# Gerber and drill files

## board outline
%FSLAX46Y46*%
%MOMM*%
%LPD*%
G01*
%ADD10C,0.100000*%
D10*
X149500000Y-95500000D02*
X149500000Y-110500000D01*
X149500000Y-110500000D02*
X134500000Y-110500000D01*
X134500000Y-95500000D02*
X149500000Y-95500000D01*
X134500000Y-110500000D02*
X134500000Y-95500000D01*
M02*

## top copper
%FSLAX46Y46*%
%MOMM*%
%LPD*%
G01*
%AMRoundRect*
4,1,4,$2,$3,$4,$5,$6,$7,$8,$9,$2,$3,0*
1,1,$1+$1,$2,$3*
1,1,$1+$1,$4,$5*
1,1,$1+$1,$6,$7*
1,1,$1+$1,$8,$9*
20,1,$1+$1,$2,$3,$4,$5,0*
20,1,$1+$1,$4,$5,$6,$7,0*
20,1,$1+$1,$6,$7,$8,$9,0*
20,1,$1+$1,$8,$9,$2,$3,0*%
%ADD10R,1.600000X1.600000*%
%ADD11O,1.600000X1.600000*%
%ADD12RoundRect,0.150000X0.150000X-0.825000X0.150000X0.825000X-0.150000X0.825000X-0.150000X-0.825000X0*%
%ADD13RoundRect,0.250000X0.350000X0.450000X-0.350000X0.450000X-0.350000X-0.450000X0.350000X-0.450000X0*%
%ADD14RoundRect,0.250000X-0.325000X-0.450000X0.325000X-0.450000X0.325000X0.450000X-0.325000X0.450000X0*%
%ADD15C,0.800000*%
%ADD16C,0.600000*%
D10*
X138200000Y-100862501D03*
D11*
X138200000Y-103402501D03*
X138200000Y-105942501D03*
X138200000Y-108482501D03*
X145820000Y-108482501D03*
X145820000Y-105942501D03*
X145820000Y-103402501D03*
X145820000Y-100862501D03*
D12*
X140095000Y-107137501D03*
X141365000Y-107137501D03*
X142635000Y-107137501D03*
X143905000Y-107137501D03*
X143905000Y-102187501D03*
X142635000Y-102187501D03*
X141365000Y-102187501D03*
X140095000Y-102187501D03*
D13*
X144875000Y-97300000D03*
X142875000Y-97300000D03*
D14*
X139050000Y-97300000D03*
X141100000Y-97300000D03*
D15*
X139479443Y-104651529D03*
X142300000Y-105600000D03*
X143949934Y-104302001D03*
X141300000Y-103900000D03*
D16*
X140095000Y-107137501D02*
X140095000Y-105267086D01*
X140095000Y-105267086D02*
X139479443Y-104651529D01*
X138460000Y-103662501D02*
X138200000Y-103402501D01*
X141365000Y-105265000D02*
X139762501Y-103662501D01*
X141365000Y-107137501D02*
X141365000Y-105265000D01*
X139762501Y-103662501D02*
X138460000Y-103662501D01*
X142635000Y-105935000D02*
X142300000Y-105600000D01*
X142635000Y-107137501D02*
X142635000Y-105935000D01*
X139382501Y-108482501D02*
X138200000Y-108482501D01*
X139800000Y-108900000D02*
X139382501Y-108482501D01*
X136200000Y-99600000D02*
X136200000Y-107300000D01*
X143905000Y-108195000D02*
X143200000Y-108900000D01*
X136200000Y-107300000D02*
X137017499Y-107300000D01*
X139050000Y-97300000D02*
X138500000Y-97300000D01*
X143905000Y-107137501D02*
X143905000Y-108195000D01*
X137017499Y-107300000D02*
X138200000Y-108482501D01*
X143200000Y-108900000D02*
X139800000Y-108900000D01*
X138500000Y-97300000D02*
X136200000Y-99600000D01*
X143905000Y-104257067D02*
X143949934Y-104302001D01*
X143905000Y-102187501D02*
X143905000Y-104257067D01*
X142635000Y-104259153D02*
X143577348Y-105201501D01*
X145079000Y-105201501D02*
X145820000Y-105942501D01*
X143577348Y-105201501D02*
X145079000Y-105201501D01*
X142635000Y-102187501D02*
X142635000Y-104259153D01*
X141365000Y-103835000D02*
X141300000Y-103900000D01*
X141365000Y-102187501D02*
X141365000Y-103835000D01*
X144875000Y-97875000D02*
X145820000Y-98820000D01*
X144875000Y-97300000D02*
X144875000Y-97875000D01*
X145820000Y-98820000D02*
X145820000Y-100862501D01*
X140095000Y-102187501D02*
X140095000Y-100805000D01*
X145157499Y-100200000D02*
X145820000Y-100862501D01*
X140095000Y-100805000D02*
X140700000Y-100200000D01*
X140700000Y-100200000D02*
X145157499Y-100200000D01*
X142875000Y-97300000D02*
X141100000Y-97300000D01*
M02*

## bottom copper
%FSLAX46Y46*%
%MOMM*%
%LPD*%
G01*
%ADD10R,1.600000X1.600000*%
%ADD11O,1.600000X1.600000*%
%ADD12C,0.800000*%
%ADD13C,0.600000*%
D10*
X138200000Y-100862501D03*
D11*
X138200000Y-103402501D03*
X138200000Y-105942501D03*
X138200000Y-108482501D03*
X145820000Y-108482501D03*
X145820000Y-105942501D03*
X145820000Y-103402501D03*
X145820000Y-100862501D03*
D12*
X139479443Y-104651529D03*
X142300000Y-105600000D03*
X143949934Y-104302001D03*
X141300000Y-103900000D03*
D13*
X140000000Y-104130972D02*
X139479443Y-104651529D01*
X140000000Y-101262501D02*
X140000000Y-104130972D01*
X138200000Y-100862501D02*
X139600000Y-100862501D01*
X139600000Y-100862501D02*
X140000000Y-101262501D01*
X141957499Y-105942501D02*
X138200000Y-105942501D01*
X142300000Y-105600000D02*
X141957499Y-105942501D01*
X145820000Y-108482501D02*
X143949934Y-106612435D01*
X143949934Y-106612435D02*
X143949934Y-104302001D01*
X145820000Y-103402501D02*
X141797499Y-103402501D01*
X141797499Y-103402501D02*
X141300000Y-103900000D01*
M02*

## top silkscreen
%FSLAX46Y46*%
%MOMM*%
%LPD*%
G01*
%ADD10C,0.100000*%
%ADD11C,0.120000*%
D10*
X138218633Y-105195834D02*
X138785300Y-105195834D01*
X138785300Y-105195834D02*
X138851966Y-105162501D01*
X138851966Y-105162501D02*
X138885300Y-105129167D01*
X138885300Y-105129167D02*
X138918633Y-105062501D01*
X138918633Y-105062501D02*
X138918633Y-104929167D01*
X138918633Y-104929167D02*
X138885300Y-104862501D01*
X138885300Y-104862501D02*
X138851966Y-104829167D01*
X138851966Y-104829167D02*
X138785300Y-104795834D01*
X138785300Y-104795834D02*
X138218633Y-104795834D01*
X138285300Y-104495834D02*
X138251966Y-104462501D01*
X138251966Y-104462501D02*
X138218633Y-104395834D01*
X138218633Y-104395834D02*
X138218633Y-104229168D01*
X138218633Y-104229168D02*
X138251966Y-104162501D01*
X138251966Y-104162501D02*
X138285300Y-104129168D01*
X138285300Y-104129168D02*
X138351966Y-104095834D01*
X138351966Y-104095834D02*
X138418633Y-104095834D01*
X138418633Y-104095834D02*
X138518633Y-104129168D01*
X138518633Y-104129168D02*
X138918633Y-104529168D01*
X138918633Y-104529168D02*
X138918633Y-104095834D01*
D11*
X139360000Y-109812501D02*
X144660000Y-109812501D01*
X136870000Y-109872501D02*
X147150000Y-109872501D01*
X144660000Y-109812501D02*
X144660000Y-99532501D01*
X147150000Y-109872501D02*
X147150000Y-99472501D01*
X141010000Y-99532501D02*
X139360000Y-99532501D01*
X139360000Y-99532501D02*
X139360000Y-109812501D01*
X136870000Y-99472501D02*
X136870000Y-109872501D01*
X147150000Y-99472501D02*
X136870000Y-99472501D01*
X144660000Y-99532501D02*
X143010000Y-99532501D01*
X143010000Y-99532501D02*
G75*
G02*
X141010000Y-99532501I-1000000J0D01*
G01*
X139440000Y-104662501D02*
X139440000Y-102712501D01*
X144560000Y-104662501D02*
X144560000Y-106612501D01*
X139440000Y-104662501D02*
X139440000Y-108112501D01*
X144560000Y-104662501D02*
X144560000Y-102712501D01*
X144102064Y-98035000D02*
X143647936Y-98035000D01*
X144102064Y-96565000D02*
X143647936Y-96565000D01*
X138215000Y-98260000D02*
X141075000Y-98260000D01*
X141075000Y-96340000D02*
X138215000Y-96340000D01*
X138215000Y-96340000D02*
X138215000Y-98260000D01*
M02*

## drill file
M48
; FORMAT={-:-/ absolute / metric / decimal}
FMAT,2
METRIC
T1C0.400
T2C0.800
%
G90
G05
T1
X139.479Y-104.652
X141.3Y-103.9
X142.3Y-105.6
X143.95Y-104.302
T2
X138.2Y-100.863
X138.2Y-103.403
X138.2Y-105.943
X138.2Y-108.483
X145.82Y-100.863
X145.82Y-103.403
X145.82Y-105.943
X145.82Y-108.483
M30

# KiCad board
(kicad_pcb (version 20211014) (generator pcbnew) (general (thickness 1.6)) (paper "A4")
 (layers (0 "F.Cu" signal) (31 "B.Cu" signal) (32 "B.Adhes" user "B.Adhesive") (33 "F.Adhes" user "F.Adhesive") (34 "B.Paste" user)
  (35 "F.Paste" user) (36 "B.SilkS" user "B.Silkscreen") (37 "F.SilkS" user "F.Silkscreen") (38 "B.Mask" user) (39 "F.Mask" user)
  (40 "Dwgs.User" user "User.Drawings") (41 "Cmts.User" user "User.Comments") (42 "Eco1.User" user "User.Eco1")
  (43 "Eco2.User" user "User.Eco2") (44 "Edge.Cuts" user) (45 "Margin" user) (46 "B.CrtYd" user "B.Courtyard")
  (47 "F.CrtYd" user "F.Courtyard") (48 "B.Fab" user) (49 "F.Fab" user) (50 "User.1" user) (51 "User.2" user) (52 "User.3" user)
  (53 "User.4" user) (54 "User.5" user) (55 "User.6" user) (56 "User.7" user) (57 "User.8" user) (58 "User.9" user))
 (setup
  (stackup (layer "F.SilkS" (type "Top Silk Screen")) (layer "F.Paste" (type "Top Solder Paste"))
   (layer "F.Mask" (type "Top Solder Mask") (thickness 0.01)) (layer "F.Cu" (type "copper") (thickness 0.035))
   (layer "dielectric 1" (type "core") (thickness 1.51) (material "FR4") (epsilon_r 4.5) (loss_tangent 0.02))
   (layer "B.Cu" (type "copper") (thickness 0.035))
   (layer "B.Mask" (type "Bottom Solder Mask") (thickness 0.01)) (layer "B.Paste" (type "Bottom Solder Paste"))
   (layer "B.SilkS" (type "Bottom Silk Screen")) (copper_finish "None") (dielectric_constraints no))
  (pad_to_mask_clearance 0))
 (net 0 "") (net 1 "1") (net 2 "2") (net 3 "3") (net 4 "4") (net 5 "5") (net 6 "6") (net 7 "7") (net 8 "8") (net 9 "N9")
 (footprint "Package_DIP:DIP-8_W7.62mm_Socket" (layer "F.Cu") (at 138.2 100.862501)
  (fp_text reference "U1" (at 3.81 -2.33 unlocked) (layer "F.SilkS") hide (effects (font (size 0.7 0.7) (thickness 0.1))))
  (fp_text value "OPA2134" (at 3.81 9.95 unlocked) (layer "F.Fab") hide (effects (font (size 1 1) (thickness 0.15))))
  (fp_line (start 1.16 8.95) (end 6.46 8.95) (layer "F.SilkS") (width 0.12))
  (fp_line (start -1.33 9.01) (end 8.95 9.01) (layer "F.SilkS") (width 0.12))
  (fp_line (start 6.46 8.95) (end 6.46 -1.33) (layer "F.SilkS") (width 0.12))
  (fp_line (start 8.95 9.01) (end 8.95 -1.39) (layer "F.SilkS") (width 0.12))
  (fp_line (start 2.81 -1.33) (end 1.16 -1.33) (layer "F.SilkS") (width 0.12))
  (fp_line (start 1.16 -1.33) (end 1.16 8.95) (layer "F.SilkS") (width 0.12))
  (fp_line (start -1.33 -1.39) (end -1.33 9.01) (layer "F.SilkS") (width 0.12))
  (fp_line (start 8.95 -1.39) (end -1.33 -1.39) (layer "F.SilkS") (width 0.12))
  (fp_line (start 6.46 -1.33) (end 4.81 -1.33) (layer "F.SilkS") (width 0.12))
  (fp_arc (start 4.81 -1.33) (mid 3.81 -0.33) (end 2.81 -1.33) (layer "F.SilkS") (width 0.12))
  (pad "1" thru_hole rect (at 0 0) (size 1.6 1.6) (drill 0.8) (layers *.Cu *.Mask) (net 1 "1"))
  (pad "2" thru_hole oval (at 0 2.54) (size 1.6 1.6) (drill 0.8) (layers *.Cu *.Mask) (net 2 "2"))
  (pad "3" thru_hole oval (at 0 5.08) (size 1.6 1.6) (drill 0.8) (layers *.Cu *.Mask) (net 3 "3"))
  (pad "4" thru_hole oval (at 0 7.62) (size 1.6 1.6) (drill 0.8) (layers *.Cu *.Mask) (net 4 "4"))
  (pad "5" thru_hole oval (at 7.62 7.62) (size 1.6 1.6) (drill 0.8) (layers *.Cu *.Mask) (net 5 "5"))
  (pad "6" thru_hole oval (at 7.62 5.08) (size 1.6 1.6) (drill 0.8) (layers *.Cu *.Mask) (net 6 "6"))
  (pad "7" thru_hole oval (at 7.62 2.54) (size 1.6 1.6) (drill 0.8) (layers *.Cu *.Mask) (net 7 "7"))
  (pad "8" thru_hole oval (at 7.62 0) (size 1.6 1.6) (drill 0.8) (layers *.Cu *.Mask) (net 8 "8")))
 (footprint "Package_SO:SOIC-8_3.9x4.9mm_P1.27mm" (layer "F.Cu") (at 142 104.662501 90)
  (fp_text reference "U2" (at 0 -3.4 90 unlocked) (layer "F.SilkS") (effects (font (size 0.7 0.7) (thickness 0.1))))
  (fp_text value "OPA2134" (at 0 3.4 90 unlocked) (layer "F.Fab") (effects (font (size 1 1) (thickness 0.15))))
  (fp_line (start 0 -2.56) (end 1.95 -2.56) (layer "F.SilkS") (width 0.12))
  (fp_line (start 0 2.56) (end -1.95 2.56) (layer "F.SilkS") (width 0.12))
  (fp_line (start 0 -2.56) (end -3.45 -2.56) (layer "F.SilkS") (width 0.12))
  (fp_line (start 0 2.56) (end 1.95 2.56) (layer "F.SilkS") (width 0.12))
  (pad "1" smd roundrect (at -2.475 -1.905 90) (size 1.95 0.6) (layers "F.Cu" "F.Paste" "F.Mask") (roundrect_rratio 0.25) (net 1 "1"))
  (pad "2" smd roundrect (at -2.475 -0.635 90) (size 1.95 0.6) (layers "F.Cu" "F.Paste" "F.Mask") (roundrect_rratio 0.25) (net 2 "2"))
  (pad "3" smd roundrect (at -2.475 0.635 90) (size 1.95 0.6) (layers "F.Cu" "F.Paste" "F.Mask") (roundrect_rratio 0.25) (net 3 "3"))
  (pad "4" smd roundrect (at -2.475 1.905 90) (size 1.95 0.6) (layers "F.Cu" "F.Paste" "F.Mask") (roundrect_rratio 0.25) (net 4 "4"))
  (pad "5" smd roundrect (at 2.475 1.905 90) (size 1.95 0.6) (layers "F.Cu" "F.Paste" "F.Mask") (roundrect_rratio 0.25) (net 5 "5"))
  (pad "6" smd roundrect (at 2.475 0.635 90) (size 1.95 0.6) (layers "F.Cu" "F.Paste" "F.Mask") (roundrect_rratio 0.25) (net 6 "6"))
  (pad "7" smd roundrect (at 2.475 -0.635 90) (size 1.95 0.6) (layers "F.Cu" "F.Paste" "F.Mask") (roundrect_rratio 0.25) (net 7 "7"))
  (pad "8" smd roundrect (at 2.475 -1.905 90) (size 1.95 0.6) (layers "F.Cu" "F.Paste" "F.Mask") (roundrect_rratio 0.25) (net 8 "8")))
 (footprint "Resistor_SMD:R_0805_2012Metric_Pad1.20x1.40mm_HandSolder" (layer "F.Cu") (at 143.875 97.3 180)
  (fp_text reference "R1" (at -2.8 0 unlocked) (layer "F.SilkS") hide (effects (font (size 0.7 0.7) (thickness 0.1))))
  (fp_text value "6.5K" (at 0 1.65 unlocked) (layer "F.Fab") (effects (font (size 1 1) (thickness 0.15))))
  (fp_line (start -0.227064 -0.735) (end 0.227064 -0.735) (layer "F.SilkS") (width 0.12))
  (fp_line (start -0.227064 0.735) (end 0.227064 0.735) (layer "F.SilkS") (width 0.12))
  (pad "1" smd roundrect (at -1 0 180) (size 1.2 1.4) (layers "F.Cu" "F.Paste" "F.Mask") (roundrect_rratio 0.208333) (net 8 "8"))
  (pad "2" smd roundrect (at 1 0 180) (size 1.2 1.4) (layers "F.Cu" "F.Paste" "F.Mask") (roundrect_rratio 0.208333) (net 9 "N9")))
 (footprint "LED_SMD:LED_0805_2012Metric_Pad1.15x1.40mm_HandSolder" (layer "F.Cu") (at 140.075 97.3)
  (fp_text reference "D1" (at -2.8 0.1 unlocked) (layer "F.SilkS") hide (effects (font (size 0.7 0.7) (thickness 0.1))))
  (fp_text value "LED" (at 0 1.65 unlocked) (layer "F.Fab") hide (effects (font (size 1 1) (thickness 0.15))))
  (fp_line (start -1.86 0.96) (end 1 0.96) (layer "F.SilkS") (width 0.12))
  (fp_line (start 1 -0.96) (end -1.86 -0.96) (layer "F.SilkS") (width 0.12))
  (fp_line (start -1.86 -0.96) (end -1.86 0.96) (layer "F.SilkS") (width 0.12))
  (pad "1" smd roundrect (at -1.025 0) (size 1.15 1.4) (layers "F.Cu" "F.Paste" "F.Mask") (roundrect_rratio 0.217391) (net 4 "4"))
  (pad "2" smd roundrect (at 1.025 0) (size 1.15 1.4) (layers "F.Cu" "F.Paste" "F.Mask") (roundrect_rratio 0.217391) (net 9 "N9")))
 (gr_line (start 149.5 95.5) (end 149.5 110.5) (layer "Edge.Cuts") (width 0.1))
 (gr_line (start 149.5 110.5) (end 134.5 110.5) (layer "Edge.Cuts") (width 0.1))
 (gr_line (start 134.5 95.5) (end 149.5 95.5) (layer "Edge.Cuts") (width 0.1))
 (gr_line (start 134.5 110.5) (end 134.5 95.5) (layer "Edge.Cuts") (width 0.1))
 (segment (start 140.095 107.137501) (end 140.095 105.267086) (width 0.6) (layer "F.Cu") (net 1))
 (segment (start 140.095 105.267086) (end 139.479443 104.651529) (width 0.6) (layer "F.Cu") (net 1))
 (via (at 139.479443 104.651529) (size 0.8) (drill 0.4) (layers "F.Cu" "B.Cu") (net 1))
 (segment (start 140 104.130972) (end 139.479443 104.651529) (width 0.6) (layer "B.Cu") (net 1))
 (segment (start 140 101.262501) (end 140 104.130972) (width 0.6) (layer "B.Cu") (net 1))
 (segment (start 138.2 100.862501) (end 139.6 100.862501) (width 0.6) (layer "B.Cu") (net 1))
 (segment (start 139.6 100.862501) (end 140 101.262501) (width 0.6) (layer "B.Cu") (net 1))
 (segment (start 138.46 103.662501) (end 138.2 103.402501) (width 0.6) (layer "F.Cu") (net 2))
 (segment (start 141.365 105.265) (end 139.762501 103.662501) (width 0.6) (layer "F.Cu") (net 2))
 (segment (start 141.365 107.137501) (end 141.365 105.265) (width 0.6) (layer "F.Cu") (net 2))
 (segment (start 139.762501 103.662501) (end 138.46 103.662501) (width 0.6) (layer "F.Cu") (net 2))
 (segment (start 142.635 105.935) (end 142.3 105.6) (width 0.6) (layer "F.Cu") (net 3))
 (segment (start 142.635 107.137501) (end 142.635 105.935) (width 0.6) (layer "F.Cu") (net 3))
 (via (at 142.3 105.6) (size 0.8) (drill 0.4) (layers "F.Cu" "B.Cu") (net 3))
 (segment (start 141.957499 105.942501) (end 138.2 105.942501) (width 0.6) (layer "B.Cu") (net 3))
 (segment (start 142.3 105.6) (end 141.957499 105.942501) (width 0.6) (layer "B.Cu") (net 3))
 (segment (start 139.382501 108.482501) (end 138.2 108.482501) (width 0.6) (layer "F.Cu") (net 4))
 (segment (start 139.8 108.9) (end 139.382501 108.482501) (width 0.6) (layer "F.Cu") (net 4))
 (segment (start 136.2 99.6) (end 136.2 107.3) (width 0.6) (layer "F.Cu") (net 4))
 (segment (start 143.905 108.195) (end 143.2 108.9) (width 0.6) (layer "F.Cu") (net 4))
 (segment (start 136.2 107.3) (end 137.017499 107.3) (width 0.6) (layer "F.Cu") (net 4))
 (segment (start 139.05 97.3) (end 138.5 97.3) (width 0.6) (layer "F.Cu") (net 4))
 (segment (start 143.905 107.137501) (end 143.905 108.195) (width 0.6) (layer "F.Cu") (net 4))
 (segment (start 137.017499 107.3) (end 138.2 108.482501) (width 0.6) (layer "F.Cu") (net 4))
 (segment (start 143.2 108.9) (end 139.8 108.9) (width 0.6) (layer "F.Cu") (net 4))
 (segment (start 138.5 97.3) (end 136.2 99.6) (width 0.6) (layer "F.Cu") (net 4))
 (segment (start 143.905 104.257067) (end 143.949934 104.302001) (width 0.6) (layer "F.Cu") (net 5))
 (segment (start 143.905 102.187501) (end 143.905 104.257067) (width 0.6) (layer "F.Cu") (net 5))
 (via (at 143.949934 104.302001) (size 0.8) (drill 0.4) (layers "F.Cu" "B.Cu") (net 5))
 (segment (start 145.82 108.482501) (end 143.949934 106.612435) (width 0.6) (layer "B.Cu") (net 5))
 (segment (start 143.949934 106.612435) (end 143.949934 104.302001) (width 0.6) (layer "B.Cu") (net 5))
 (segment (start 142.635 104.259153) (end 143.577348 105.201501) (width 0.6) (layer "F.Cu") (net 6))
 (segment (start 145.079 105.201501) (end 145.82 105.942501) (width 0.6) (layer "F.Cu") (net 6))
 (segment (start 143.577348 105.201501) (end 145.079 105.201501) (width 0.6) (layer "F.Cu") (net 6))
 (segment (start 142.635 102.187501) (end 142.635 104.259153) (width 0.6) (layer "F.Cu") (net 6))
 (segment (start 141.365 103.835) (end 141.3 103.9) (width 0.6) (layer "F.Cu") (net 7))
 (segment (start 141.365 102.187501) (end 141.365 103.835) (width 0.6) (layer "F.Cu") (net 7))
 (via (at 141.3 103.9) (size 0.8) (drill 0.4) (layers "F.Cu" "B.Cu") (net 7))
 (segment (start 145.82 103.402501) (end 141.797499 103.402501) (width 0.6) (layer "B.Cu") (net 7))
 (segment (start 141.797499 103.402501) (end 141.3 103.9) (width 0.6) (layer "B.Cu") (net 7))
 (segment (start 144.875 97.875) (end 145.82 98.82) (width 0.6) (layer "F.Cu") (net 8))
 (segment (start 144.875 97.3) (end 144.875 97.875) (width 0.6) (layer "F.Cu") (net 8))
 (segment (start 145.82 98.82) (end 145.82 100.862501) (width 0.6) (layer "F.Cu") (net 8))
 (segment (start 140.095 102.187501) (end 140.095 100.805) (width 0.6) (layer "F.Cu") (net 8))
 (segment (start 145.157499 100.2) (end 145.82 100.862501) (width 0.6) (layer "F.Cu") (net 8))
 (segment (start 140.095 100.805) (end 140.7 100.2) (width 0.6) (layer "F.Cu") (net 8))
 (segment (start 140.7 100.2) (end 145.157499 100.2) (width 0.6) (layer "F.Cu") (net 8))
 (segment (start 142.875 97.3) (end 141.1 97.3) (width 0.6) (layer "F.Cu") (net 9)))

